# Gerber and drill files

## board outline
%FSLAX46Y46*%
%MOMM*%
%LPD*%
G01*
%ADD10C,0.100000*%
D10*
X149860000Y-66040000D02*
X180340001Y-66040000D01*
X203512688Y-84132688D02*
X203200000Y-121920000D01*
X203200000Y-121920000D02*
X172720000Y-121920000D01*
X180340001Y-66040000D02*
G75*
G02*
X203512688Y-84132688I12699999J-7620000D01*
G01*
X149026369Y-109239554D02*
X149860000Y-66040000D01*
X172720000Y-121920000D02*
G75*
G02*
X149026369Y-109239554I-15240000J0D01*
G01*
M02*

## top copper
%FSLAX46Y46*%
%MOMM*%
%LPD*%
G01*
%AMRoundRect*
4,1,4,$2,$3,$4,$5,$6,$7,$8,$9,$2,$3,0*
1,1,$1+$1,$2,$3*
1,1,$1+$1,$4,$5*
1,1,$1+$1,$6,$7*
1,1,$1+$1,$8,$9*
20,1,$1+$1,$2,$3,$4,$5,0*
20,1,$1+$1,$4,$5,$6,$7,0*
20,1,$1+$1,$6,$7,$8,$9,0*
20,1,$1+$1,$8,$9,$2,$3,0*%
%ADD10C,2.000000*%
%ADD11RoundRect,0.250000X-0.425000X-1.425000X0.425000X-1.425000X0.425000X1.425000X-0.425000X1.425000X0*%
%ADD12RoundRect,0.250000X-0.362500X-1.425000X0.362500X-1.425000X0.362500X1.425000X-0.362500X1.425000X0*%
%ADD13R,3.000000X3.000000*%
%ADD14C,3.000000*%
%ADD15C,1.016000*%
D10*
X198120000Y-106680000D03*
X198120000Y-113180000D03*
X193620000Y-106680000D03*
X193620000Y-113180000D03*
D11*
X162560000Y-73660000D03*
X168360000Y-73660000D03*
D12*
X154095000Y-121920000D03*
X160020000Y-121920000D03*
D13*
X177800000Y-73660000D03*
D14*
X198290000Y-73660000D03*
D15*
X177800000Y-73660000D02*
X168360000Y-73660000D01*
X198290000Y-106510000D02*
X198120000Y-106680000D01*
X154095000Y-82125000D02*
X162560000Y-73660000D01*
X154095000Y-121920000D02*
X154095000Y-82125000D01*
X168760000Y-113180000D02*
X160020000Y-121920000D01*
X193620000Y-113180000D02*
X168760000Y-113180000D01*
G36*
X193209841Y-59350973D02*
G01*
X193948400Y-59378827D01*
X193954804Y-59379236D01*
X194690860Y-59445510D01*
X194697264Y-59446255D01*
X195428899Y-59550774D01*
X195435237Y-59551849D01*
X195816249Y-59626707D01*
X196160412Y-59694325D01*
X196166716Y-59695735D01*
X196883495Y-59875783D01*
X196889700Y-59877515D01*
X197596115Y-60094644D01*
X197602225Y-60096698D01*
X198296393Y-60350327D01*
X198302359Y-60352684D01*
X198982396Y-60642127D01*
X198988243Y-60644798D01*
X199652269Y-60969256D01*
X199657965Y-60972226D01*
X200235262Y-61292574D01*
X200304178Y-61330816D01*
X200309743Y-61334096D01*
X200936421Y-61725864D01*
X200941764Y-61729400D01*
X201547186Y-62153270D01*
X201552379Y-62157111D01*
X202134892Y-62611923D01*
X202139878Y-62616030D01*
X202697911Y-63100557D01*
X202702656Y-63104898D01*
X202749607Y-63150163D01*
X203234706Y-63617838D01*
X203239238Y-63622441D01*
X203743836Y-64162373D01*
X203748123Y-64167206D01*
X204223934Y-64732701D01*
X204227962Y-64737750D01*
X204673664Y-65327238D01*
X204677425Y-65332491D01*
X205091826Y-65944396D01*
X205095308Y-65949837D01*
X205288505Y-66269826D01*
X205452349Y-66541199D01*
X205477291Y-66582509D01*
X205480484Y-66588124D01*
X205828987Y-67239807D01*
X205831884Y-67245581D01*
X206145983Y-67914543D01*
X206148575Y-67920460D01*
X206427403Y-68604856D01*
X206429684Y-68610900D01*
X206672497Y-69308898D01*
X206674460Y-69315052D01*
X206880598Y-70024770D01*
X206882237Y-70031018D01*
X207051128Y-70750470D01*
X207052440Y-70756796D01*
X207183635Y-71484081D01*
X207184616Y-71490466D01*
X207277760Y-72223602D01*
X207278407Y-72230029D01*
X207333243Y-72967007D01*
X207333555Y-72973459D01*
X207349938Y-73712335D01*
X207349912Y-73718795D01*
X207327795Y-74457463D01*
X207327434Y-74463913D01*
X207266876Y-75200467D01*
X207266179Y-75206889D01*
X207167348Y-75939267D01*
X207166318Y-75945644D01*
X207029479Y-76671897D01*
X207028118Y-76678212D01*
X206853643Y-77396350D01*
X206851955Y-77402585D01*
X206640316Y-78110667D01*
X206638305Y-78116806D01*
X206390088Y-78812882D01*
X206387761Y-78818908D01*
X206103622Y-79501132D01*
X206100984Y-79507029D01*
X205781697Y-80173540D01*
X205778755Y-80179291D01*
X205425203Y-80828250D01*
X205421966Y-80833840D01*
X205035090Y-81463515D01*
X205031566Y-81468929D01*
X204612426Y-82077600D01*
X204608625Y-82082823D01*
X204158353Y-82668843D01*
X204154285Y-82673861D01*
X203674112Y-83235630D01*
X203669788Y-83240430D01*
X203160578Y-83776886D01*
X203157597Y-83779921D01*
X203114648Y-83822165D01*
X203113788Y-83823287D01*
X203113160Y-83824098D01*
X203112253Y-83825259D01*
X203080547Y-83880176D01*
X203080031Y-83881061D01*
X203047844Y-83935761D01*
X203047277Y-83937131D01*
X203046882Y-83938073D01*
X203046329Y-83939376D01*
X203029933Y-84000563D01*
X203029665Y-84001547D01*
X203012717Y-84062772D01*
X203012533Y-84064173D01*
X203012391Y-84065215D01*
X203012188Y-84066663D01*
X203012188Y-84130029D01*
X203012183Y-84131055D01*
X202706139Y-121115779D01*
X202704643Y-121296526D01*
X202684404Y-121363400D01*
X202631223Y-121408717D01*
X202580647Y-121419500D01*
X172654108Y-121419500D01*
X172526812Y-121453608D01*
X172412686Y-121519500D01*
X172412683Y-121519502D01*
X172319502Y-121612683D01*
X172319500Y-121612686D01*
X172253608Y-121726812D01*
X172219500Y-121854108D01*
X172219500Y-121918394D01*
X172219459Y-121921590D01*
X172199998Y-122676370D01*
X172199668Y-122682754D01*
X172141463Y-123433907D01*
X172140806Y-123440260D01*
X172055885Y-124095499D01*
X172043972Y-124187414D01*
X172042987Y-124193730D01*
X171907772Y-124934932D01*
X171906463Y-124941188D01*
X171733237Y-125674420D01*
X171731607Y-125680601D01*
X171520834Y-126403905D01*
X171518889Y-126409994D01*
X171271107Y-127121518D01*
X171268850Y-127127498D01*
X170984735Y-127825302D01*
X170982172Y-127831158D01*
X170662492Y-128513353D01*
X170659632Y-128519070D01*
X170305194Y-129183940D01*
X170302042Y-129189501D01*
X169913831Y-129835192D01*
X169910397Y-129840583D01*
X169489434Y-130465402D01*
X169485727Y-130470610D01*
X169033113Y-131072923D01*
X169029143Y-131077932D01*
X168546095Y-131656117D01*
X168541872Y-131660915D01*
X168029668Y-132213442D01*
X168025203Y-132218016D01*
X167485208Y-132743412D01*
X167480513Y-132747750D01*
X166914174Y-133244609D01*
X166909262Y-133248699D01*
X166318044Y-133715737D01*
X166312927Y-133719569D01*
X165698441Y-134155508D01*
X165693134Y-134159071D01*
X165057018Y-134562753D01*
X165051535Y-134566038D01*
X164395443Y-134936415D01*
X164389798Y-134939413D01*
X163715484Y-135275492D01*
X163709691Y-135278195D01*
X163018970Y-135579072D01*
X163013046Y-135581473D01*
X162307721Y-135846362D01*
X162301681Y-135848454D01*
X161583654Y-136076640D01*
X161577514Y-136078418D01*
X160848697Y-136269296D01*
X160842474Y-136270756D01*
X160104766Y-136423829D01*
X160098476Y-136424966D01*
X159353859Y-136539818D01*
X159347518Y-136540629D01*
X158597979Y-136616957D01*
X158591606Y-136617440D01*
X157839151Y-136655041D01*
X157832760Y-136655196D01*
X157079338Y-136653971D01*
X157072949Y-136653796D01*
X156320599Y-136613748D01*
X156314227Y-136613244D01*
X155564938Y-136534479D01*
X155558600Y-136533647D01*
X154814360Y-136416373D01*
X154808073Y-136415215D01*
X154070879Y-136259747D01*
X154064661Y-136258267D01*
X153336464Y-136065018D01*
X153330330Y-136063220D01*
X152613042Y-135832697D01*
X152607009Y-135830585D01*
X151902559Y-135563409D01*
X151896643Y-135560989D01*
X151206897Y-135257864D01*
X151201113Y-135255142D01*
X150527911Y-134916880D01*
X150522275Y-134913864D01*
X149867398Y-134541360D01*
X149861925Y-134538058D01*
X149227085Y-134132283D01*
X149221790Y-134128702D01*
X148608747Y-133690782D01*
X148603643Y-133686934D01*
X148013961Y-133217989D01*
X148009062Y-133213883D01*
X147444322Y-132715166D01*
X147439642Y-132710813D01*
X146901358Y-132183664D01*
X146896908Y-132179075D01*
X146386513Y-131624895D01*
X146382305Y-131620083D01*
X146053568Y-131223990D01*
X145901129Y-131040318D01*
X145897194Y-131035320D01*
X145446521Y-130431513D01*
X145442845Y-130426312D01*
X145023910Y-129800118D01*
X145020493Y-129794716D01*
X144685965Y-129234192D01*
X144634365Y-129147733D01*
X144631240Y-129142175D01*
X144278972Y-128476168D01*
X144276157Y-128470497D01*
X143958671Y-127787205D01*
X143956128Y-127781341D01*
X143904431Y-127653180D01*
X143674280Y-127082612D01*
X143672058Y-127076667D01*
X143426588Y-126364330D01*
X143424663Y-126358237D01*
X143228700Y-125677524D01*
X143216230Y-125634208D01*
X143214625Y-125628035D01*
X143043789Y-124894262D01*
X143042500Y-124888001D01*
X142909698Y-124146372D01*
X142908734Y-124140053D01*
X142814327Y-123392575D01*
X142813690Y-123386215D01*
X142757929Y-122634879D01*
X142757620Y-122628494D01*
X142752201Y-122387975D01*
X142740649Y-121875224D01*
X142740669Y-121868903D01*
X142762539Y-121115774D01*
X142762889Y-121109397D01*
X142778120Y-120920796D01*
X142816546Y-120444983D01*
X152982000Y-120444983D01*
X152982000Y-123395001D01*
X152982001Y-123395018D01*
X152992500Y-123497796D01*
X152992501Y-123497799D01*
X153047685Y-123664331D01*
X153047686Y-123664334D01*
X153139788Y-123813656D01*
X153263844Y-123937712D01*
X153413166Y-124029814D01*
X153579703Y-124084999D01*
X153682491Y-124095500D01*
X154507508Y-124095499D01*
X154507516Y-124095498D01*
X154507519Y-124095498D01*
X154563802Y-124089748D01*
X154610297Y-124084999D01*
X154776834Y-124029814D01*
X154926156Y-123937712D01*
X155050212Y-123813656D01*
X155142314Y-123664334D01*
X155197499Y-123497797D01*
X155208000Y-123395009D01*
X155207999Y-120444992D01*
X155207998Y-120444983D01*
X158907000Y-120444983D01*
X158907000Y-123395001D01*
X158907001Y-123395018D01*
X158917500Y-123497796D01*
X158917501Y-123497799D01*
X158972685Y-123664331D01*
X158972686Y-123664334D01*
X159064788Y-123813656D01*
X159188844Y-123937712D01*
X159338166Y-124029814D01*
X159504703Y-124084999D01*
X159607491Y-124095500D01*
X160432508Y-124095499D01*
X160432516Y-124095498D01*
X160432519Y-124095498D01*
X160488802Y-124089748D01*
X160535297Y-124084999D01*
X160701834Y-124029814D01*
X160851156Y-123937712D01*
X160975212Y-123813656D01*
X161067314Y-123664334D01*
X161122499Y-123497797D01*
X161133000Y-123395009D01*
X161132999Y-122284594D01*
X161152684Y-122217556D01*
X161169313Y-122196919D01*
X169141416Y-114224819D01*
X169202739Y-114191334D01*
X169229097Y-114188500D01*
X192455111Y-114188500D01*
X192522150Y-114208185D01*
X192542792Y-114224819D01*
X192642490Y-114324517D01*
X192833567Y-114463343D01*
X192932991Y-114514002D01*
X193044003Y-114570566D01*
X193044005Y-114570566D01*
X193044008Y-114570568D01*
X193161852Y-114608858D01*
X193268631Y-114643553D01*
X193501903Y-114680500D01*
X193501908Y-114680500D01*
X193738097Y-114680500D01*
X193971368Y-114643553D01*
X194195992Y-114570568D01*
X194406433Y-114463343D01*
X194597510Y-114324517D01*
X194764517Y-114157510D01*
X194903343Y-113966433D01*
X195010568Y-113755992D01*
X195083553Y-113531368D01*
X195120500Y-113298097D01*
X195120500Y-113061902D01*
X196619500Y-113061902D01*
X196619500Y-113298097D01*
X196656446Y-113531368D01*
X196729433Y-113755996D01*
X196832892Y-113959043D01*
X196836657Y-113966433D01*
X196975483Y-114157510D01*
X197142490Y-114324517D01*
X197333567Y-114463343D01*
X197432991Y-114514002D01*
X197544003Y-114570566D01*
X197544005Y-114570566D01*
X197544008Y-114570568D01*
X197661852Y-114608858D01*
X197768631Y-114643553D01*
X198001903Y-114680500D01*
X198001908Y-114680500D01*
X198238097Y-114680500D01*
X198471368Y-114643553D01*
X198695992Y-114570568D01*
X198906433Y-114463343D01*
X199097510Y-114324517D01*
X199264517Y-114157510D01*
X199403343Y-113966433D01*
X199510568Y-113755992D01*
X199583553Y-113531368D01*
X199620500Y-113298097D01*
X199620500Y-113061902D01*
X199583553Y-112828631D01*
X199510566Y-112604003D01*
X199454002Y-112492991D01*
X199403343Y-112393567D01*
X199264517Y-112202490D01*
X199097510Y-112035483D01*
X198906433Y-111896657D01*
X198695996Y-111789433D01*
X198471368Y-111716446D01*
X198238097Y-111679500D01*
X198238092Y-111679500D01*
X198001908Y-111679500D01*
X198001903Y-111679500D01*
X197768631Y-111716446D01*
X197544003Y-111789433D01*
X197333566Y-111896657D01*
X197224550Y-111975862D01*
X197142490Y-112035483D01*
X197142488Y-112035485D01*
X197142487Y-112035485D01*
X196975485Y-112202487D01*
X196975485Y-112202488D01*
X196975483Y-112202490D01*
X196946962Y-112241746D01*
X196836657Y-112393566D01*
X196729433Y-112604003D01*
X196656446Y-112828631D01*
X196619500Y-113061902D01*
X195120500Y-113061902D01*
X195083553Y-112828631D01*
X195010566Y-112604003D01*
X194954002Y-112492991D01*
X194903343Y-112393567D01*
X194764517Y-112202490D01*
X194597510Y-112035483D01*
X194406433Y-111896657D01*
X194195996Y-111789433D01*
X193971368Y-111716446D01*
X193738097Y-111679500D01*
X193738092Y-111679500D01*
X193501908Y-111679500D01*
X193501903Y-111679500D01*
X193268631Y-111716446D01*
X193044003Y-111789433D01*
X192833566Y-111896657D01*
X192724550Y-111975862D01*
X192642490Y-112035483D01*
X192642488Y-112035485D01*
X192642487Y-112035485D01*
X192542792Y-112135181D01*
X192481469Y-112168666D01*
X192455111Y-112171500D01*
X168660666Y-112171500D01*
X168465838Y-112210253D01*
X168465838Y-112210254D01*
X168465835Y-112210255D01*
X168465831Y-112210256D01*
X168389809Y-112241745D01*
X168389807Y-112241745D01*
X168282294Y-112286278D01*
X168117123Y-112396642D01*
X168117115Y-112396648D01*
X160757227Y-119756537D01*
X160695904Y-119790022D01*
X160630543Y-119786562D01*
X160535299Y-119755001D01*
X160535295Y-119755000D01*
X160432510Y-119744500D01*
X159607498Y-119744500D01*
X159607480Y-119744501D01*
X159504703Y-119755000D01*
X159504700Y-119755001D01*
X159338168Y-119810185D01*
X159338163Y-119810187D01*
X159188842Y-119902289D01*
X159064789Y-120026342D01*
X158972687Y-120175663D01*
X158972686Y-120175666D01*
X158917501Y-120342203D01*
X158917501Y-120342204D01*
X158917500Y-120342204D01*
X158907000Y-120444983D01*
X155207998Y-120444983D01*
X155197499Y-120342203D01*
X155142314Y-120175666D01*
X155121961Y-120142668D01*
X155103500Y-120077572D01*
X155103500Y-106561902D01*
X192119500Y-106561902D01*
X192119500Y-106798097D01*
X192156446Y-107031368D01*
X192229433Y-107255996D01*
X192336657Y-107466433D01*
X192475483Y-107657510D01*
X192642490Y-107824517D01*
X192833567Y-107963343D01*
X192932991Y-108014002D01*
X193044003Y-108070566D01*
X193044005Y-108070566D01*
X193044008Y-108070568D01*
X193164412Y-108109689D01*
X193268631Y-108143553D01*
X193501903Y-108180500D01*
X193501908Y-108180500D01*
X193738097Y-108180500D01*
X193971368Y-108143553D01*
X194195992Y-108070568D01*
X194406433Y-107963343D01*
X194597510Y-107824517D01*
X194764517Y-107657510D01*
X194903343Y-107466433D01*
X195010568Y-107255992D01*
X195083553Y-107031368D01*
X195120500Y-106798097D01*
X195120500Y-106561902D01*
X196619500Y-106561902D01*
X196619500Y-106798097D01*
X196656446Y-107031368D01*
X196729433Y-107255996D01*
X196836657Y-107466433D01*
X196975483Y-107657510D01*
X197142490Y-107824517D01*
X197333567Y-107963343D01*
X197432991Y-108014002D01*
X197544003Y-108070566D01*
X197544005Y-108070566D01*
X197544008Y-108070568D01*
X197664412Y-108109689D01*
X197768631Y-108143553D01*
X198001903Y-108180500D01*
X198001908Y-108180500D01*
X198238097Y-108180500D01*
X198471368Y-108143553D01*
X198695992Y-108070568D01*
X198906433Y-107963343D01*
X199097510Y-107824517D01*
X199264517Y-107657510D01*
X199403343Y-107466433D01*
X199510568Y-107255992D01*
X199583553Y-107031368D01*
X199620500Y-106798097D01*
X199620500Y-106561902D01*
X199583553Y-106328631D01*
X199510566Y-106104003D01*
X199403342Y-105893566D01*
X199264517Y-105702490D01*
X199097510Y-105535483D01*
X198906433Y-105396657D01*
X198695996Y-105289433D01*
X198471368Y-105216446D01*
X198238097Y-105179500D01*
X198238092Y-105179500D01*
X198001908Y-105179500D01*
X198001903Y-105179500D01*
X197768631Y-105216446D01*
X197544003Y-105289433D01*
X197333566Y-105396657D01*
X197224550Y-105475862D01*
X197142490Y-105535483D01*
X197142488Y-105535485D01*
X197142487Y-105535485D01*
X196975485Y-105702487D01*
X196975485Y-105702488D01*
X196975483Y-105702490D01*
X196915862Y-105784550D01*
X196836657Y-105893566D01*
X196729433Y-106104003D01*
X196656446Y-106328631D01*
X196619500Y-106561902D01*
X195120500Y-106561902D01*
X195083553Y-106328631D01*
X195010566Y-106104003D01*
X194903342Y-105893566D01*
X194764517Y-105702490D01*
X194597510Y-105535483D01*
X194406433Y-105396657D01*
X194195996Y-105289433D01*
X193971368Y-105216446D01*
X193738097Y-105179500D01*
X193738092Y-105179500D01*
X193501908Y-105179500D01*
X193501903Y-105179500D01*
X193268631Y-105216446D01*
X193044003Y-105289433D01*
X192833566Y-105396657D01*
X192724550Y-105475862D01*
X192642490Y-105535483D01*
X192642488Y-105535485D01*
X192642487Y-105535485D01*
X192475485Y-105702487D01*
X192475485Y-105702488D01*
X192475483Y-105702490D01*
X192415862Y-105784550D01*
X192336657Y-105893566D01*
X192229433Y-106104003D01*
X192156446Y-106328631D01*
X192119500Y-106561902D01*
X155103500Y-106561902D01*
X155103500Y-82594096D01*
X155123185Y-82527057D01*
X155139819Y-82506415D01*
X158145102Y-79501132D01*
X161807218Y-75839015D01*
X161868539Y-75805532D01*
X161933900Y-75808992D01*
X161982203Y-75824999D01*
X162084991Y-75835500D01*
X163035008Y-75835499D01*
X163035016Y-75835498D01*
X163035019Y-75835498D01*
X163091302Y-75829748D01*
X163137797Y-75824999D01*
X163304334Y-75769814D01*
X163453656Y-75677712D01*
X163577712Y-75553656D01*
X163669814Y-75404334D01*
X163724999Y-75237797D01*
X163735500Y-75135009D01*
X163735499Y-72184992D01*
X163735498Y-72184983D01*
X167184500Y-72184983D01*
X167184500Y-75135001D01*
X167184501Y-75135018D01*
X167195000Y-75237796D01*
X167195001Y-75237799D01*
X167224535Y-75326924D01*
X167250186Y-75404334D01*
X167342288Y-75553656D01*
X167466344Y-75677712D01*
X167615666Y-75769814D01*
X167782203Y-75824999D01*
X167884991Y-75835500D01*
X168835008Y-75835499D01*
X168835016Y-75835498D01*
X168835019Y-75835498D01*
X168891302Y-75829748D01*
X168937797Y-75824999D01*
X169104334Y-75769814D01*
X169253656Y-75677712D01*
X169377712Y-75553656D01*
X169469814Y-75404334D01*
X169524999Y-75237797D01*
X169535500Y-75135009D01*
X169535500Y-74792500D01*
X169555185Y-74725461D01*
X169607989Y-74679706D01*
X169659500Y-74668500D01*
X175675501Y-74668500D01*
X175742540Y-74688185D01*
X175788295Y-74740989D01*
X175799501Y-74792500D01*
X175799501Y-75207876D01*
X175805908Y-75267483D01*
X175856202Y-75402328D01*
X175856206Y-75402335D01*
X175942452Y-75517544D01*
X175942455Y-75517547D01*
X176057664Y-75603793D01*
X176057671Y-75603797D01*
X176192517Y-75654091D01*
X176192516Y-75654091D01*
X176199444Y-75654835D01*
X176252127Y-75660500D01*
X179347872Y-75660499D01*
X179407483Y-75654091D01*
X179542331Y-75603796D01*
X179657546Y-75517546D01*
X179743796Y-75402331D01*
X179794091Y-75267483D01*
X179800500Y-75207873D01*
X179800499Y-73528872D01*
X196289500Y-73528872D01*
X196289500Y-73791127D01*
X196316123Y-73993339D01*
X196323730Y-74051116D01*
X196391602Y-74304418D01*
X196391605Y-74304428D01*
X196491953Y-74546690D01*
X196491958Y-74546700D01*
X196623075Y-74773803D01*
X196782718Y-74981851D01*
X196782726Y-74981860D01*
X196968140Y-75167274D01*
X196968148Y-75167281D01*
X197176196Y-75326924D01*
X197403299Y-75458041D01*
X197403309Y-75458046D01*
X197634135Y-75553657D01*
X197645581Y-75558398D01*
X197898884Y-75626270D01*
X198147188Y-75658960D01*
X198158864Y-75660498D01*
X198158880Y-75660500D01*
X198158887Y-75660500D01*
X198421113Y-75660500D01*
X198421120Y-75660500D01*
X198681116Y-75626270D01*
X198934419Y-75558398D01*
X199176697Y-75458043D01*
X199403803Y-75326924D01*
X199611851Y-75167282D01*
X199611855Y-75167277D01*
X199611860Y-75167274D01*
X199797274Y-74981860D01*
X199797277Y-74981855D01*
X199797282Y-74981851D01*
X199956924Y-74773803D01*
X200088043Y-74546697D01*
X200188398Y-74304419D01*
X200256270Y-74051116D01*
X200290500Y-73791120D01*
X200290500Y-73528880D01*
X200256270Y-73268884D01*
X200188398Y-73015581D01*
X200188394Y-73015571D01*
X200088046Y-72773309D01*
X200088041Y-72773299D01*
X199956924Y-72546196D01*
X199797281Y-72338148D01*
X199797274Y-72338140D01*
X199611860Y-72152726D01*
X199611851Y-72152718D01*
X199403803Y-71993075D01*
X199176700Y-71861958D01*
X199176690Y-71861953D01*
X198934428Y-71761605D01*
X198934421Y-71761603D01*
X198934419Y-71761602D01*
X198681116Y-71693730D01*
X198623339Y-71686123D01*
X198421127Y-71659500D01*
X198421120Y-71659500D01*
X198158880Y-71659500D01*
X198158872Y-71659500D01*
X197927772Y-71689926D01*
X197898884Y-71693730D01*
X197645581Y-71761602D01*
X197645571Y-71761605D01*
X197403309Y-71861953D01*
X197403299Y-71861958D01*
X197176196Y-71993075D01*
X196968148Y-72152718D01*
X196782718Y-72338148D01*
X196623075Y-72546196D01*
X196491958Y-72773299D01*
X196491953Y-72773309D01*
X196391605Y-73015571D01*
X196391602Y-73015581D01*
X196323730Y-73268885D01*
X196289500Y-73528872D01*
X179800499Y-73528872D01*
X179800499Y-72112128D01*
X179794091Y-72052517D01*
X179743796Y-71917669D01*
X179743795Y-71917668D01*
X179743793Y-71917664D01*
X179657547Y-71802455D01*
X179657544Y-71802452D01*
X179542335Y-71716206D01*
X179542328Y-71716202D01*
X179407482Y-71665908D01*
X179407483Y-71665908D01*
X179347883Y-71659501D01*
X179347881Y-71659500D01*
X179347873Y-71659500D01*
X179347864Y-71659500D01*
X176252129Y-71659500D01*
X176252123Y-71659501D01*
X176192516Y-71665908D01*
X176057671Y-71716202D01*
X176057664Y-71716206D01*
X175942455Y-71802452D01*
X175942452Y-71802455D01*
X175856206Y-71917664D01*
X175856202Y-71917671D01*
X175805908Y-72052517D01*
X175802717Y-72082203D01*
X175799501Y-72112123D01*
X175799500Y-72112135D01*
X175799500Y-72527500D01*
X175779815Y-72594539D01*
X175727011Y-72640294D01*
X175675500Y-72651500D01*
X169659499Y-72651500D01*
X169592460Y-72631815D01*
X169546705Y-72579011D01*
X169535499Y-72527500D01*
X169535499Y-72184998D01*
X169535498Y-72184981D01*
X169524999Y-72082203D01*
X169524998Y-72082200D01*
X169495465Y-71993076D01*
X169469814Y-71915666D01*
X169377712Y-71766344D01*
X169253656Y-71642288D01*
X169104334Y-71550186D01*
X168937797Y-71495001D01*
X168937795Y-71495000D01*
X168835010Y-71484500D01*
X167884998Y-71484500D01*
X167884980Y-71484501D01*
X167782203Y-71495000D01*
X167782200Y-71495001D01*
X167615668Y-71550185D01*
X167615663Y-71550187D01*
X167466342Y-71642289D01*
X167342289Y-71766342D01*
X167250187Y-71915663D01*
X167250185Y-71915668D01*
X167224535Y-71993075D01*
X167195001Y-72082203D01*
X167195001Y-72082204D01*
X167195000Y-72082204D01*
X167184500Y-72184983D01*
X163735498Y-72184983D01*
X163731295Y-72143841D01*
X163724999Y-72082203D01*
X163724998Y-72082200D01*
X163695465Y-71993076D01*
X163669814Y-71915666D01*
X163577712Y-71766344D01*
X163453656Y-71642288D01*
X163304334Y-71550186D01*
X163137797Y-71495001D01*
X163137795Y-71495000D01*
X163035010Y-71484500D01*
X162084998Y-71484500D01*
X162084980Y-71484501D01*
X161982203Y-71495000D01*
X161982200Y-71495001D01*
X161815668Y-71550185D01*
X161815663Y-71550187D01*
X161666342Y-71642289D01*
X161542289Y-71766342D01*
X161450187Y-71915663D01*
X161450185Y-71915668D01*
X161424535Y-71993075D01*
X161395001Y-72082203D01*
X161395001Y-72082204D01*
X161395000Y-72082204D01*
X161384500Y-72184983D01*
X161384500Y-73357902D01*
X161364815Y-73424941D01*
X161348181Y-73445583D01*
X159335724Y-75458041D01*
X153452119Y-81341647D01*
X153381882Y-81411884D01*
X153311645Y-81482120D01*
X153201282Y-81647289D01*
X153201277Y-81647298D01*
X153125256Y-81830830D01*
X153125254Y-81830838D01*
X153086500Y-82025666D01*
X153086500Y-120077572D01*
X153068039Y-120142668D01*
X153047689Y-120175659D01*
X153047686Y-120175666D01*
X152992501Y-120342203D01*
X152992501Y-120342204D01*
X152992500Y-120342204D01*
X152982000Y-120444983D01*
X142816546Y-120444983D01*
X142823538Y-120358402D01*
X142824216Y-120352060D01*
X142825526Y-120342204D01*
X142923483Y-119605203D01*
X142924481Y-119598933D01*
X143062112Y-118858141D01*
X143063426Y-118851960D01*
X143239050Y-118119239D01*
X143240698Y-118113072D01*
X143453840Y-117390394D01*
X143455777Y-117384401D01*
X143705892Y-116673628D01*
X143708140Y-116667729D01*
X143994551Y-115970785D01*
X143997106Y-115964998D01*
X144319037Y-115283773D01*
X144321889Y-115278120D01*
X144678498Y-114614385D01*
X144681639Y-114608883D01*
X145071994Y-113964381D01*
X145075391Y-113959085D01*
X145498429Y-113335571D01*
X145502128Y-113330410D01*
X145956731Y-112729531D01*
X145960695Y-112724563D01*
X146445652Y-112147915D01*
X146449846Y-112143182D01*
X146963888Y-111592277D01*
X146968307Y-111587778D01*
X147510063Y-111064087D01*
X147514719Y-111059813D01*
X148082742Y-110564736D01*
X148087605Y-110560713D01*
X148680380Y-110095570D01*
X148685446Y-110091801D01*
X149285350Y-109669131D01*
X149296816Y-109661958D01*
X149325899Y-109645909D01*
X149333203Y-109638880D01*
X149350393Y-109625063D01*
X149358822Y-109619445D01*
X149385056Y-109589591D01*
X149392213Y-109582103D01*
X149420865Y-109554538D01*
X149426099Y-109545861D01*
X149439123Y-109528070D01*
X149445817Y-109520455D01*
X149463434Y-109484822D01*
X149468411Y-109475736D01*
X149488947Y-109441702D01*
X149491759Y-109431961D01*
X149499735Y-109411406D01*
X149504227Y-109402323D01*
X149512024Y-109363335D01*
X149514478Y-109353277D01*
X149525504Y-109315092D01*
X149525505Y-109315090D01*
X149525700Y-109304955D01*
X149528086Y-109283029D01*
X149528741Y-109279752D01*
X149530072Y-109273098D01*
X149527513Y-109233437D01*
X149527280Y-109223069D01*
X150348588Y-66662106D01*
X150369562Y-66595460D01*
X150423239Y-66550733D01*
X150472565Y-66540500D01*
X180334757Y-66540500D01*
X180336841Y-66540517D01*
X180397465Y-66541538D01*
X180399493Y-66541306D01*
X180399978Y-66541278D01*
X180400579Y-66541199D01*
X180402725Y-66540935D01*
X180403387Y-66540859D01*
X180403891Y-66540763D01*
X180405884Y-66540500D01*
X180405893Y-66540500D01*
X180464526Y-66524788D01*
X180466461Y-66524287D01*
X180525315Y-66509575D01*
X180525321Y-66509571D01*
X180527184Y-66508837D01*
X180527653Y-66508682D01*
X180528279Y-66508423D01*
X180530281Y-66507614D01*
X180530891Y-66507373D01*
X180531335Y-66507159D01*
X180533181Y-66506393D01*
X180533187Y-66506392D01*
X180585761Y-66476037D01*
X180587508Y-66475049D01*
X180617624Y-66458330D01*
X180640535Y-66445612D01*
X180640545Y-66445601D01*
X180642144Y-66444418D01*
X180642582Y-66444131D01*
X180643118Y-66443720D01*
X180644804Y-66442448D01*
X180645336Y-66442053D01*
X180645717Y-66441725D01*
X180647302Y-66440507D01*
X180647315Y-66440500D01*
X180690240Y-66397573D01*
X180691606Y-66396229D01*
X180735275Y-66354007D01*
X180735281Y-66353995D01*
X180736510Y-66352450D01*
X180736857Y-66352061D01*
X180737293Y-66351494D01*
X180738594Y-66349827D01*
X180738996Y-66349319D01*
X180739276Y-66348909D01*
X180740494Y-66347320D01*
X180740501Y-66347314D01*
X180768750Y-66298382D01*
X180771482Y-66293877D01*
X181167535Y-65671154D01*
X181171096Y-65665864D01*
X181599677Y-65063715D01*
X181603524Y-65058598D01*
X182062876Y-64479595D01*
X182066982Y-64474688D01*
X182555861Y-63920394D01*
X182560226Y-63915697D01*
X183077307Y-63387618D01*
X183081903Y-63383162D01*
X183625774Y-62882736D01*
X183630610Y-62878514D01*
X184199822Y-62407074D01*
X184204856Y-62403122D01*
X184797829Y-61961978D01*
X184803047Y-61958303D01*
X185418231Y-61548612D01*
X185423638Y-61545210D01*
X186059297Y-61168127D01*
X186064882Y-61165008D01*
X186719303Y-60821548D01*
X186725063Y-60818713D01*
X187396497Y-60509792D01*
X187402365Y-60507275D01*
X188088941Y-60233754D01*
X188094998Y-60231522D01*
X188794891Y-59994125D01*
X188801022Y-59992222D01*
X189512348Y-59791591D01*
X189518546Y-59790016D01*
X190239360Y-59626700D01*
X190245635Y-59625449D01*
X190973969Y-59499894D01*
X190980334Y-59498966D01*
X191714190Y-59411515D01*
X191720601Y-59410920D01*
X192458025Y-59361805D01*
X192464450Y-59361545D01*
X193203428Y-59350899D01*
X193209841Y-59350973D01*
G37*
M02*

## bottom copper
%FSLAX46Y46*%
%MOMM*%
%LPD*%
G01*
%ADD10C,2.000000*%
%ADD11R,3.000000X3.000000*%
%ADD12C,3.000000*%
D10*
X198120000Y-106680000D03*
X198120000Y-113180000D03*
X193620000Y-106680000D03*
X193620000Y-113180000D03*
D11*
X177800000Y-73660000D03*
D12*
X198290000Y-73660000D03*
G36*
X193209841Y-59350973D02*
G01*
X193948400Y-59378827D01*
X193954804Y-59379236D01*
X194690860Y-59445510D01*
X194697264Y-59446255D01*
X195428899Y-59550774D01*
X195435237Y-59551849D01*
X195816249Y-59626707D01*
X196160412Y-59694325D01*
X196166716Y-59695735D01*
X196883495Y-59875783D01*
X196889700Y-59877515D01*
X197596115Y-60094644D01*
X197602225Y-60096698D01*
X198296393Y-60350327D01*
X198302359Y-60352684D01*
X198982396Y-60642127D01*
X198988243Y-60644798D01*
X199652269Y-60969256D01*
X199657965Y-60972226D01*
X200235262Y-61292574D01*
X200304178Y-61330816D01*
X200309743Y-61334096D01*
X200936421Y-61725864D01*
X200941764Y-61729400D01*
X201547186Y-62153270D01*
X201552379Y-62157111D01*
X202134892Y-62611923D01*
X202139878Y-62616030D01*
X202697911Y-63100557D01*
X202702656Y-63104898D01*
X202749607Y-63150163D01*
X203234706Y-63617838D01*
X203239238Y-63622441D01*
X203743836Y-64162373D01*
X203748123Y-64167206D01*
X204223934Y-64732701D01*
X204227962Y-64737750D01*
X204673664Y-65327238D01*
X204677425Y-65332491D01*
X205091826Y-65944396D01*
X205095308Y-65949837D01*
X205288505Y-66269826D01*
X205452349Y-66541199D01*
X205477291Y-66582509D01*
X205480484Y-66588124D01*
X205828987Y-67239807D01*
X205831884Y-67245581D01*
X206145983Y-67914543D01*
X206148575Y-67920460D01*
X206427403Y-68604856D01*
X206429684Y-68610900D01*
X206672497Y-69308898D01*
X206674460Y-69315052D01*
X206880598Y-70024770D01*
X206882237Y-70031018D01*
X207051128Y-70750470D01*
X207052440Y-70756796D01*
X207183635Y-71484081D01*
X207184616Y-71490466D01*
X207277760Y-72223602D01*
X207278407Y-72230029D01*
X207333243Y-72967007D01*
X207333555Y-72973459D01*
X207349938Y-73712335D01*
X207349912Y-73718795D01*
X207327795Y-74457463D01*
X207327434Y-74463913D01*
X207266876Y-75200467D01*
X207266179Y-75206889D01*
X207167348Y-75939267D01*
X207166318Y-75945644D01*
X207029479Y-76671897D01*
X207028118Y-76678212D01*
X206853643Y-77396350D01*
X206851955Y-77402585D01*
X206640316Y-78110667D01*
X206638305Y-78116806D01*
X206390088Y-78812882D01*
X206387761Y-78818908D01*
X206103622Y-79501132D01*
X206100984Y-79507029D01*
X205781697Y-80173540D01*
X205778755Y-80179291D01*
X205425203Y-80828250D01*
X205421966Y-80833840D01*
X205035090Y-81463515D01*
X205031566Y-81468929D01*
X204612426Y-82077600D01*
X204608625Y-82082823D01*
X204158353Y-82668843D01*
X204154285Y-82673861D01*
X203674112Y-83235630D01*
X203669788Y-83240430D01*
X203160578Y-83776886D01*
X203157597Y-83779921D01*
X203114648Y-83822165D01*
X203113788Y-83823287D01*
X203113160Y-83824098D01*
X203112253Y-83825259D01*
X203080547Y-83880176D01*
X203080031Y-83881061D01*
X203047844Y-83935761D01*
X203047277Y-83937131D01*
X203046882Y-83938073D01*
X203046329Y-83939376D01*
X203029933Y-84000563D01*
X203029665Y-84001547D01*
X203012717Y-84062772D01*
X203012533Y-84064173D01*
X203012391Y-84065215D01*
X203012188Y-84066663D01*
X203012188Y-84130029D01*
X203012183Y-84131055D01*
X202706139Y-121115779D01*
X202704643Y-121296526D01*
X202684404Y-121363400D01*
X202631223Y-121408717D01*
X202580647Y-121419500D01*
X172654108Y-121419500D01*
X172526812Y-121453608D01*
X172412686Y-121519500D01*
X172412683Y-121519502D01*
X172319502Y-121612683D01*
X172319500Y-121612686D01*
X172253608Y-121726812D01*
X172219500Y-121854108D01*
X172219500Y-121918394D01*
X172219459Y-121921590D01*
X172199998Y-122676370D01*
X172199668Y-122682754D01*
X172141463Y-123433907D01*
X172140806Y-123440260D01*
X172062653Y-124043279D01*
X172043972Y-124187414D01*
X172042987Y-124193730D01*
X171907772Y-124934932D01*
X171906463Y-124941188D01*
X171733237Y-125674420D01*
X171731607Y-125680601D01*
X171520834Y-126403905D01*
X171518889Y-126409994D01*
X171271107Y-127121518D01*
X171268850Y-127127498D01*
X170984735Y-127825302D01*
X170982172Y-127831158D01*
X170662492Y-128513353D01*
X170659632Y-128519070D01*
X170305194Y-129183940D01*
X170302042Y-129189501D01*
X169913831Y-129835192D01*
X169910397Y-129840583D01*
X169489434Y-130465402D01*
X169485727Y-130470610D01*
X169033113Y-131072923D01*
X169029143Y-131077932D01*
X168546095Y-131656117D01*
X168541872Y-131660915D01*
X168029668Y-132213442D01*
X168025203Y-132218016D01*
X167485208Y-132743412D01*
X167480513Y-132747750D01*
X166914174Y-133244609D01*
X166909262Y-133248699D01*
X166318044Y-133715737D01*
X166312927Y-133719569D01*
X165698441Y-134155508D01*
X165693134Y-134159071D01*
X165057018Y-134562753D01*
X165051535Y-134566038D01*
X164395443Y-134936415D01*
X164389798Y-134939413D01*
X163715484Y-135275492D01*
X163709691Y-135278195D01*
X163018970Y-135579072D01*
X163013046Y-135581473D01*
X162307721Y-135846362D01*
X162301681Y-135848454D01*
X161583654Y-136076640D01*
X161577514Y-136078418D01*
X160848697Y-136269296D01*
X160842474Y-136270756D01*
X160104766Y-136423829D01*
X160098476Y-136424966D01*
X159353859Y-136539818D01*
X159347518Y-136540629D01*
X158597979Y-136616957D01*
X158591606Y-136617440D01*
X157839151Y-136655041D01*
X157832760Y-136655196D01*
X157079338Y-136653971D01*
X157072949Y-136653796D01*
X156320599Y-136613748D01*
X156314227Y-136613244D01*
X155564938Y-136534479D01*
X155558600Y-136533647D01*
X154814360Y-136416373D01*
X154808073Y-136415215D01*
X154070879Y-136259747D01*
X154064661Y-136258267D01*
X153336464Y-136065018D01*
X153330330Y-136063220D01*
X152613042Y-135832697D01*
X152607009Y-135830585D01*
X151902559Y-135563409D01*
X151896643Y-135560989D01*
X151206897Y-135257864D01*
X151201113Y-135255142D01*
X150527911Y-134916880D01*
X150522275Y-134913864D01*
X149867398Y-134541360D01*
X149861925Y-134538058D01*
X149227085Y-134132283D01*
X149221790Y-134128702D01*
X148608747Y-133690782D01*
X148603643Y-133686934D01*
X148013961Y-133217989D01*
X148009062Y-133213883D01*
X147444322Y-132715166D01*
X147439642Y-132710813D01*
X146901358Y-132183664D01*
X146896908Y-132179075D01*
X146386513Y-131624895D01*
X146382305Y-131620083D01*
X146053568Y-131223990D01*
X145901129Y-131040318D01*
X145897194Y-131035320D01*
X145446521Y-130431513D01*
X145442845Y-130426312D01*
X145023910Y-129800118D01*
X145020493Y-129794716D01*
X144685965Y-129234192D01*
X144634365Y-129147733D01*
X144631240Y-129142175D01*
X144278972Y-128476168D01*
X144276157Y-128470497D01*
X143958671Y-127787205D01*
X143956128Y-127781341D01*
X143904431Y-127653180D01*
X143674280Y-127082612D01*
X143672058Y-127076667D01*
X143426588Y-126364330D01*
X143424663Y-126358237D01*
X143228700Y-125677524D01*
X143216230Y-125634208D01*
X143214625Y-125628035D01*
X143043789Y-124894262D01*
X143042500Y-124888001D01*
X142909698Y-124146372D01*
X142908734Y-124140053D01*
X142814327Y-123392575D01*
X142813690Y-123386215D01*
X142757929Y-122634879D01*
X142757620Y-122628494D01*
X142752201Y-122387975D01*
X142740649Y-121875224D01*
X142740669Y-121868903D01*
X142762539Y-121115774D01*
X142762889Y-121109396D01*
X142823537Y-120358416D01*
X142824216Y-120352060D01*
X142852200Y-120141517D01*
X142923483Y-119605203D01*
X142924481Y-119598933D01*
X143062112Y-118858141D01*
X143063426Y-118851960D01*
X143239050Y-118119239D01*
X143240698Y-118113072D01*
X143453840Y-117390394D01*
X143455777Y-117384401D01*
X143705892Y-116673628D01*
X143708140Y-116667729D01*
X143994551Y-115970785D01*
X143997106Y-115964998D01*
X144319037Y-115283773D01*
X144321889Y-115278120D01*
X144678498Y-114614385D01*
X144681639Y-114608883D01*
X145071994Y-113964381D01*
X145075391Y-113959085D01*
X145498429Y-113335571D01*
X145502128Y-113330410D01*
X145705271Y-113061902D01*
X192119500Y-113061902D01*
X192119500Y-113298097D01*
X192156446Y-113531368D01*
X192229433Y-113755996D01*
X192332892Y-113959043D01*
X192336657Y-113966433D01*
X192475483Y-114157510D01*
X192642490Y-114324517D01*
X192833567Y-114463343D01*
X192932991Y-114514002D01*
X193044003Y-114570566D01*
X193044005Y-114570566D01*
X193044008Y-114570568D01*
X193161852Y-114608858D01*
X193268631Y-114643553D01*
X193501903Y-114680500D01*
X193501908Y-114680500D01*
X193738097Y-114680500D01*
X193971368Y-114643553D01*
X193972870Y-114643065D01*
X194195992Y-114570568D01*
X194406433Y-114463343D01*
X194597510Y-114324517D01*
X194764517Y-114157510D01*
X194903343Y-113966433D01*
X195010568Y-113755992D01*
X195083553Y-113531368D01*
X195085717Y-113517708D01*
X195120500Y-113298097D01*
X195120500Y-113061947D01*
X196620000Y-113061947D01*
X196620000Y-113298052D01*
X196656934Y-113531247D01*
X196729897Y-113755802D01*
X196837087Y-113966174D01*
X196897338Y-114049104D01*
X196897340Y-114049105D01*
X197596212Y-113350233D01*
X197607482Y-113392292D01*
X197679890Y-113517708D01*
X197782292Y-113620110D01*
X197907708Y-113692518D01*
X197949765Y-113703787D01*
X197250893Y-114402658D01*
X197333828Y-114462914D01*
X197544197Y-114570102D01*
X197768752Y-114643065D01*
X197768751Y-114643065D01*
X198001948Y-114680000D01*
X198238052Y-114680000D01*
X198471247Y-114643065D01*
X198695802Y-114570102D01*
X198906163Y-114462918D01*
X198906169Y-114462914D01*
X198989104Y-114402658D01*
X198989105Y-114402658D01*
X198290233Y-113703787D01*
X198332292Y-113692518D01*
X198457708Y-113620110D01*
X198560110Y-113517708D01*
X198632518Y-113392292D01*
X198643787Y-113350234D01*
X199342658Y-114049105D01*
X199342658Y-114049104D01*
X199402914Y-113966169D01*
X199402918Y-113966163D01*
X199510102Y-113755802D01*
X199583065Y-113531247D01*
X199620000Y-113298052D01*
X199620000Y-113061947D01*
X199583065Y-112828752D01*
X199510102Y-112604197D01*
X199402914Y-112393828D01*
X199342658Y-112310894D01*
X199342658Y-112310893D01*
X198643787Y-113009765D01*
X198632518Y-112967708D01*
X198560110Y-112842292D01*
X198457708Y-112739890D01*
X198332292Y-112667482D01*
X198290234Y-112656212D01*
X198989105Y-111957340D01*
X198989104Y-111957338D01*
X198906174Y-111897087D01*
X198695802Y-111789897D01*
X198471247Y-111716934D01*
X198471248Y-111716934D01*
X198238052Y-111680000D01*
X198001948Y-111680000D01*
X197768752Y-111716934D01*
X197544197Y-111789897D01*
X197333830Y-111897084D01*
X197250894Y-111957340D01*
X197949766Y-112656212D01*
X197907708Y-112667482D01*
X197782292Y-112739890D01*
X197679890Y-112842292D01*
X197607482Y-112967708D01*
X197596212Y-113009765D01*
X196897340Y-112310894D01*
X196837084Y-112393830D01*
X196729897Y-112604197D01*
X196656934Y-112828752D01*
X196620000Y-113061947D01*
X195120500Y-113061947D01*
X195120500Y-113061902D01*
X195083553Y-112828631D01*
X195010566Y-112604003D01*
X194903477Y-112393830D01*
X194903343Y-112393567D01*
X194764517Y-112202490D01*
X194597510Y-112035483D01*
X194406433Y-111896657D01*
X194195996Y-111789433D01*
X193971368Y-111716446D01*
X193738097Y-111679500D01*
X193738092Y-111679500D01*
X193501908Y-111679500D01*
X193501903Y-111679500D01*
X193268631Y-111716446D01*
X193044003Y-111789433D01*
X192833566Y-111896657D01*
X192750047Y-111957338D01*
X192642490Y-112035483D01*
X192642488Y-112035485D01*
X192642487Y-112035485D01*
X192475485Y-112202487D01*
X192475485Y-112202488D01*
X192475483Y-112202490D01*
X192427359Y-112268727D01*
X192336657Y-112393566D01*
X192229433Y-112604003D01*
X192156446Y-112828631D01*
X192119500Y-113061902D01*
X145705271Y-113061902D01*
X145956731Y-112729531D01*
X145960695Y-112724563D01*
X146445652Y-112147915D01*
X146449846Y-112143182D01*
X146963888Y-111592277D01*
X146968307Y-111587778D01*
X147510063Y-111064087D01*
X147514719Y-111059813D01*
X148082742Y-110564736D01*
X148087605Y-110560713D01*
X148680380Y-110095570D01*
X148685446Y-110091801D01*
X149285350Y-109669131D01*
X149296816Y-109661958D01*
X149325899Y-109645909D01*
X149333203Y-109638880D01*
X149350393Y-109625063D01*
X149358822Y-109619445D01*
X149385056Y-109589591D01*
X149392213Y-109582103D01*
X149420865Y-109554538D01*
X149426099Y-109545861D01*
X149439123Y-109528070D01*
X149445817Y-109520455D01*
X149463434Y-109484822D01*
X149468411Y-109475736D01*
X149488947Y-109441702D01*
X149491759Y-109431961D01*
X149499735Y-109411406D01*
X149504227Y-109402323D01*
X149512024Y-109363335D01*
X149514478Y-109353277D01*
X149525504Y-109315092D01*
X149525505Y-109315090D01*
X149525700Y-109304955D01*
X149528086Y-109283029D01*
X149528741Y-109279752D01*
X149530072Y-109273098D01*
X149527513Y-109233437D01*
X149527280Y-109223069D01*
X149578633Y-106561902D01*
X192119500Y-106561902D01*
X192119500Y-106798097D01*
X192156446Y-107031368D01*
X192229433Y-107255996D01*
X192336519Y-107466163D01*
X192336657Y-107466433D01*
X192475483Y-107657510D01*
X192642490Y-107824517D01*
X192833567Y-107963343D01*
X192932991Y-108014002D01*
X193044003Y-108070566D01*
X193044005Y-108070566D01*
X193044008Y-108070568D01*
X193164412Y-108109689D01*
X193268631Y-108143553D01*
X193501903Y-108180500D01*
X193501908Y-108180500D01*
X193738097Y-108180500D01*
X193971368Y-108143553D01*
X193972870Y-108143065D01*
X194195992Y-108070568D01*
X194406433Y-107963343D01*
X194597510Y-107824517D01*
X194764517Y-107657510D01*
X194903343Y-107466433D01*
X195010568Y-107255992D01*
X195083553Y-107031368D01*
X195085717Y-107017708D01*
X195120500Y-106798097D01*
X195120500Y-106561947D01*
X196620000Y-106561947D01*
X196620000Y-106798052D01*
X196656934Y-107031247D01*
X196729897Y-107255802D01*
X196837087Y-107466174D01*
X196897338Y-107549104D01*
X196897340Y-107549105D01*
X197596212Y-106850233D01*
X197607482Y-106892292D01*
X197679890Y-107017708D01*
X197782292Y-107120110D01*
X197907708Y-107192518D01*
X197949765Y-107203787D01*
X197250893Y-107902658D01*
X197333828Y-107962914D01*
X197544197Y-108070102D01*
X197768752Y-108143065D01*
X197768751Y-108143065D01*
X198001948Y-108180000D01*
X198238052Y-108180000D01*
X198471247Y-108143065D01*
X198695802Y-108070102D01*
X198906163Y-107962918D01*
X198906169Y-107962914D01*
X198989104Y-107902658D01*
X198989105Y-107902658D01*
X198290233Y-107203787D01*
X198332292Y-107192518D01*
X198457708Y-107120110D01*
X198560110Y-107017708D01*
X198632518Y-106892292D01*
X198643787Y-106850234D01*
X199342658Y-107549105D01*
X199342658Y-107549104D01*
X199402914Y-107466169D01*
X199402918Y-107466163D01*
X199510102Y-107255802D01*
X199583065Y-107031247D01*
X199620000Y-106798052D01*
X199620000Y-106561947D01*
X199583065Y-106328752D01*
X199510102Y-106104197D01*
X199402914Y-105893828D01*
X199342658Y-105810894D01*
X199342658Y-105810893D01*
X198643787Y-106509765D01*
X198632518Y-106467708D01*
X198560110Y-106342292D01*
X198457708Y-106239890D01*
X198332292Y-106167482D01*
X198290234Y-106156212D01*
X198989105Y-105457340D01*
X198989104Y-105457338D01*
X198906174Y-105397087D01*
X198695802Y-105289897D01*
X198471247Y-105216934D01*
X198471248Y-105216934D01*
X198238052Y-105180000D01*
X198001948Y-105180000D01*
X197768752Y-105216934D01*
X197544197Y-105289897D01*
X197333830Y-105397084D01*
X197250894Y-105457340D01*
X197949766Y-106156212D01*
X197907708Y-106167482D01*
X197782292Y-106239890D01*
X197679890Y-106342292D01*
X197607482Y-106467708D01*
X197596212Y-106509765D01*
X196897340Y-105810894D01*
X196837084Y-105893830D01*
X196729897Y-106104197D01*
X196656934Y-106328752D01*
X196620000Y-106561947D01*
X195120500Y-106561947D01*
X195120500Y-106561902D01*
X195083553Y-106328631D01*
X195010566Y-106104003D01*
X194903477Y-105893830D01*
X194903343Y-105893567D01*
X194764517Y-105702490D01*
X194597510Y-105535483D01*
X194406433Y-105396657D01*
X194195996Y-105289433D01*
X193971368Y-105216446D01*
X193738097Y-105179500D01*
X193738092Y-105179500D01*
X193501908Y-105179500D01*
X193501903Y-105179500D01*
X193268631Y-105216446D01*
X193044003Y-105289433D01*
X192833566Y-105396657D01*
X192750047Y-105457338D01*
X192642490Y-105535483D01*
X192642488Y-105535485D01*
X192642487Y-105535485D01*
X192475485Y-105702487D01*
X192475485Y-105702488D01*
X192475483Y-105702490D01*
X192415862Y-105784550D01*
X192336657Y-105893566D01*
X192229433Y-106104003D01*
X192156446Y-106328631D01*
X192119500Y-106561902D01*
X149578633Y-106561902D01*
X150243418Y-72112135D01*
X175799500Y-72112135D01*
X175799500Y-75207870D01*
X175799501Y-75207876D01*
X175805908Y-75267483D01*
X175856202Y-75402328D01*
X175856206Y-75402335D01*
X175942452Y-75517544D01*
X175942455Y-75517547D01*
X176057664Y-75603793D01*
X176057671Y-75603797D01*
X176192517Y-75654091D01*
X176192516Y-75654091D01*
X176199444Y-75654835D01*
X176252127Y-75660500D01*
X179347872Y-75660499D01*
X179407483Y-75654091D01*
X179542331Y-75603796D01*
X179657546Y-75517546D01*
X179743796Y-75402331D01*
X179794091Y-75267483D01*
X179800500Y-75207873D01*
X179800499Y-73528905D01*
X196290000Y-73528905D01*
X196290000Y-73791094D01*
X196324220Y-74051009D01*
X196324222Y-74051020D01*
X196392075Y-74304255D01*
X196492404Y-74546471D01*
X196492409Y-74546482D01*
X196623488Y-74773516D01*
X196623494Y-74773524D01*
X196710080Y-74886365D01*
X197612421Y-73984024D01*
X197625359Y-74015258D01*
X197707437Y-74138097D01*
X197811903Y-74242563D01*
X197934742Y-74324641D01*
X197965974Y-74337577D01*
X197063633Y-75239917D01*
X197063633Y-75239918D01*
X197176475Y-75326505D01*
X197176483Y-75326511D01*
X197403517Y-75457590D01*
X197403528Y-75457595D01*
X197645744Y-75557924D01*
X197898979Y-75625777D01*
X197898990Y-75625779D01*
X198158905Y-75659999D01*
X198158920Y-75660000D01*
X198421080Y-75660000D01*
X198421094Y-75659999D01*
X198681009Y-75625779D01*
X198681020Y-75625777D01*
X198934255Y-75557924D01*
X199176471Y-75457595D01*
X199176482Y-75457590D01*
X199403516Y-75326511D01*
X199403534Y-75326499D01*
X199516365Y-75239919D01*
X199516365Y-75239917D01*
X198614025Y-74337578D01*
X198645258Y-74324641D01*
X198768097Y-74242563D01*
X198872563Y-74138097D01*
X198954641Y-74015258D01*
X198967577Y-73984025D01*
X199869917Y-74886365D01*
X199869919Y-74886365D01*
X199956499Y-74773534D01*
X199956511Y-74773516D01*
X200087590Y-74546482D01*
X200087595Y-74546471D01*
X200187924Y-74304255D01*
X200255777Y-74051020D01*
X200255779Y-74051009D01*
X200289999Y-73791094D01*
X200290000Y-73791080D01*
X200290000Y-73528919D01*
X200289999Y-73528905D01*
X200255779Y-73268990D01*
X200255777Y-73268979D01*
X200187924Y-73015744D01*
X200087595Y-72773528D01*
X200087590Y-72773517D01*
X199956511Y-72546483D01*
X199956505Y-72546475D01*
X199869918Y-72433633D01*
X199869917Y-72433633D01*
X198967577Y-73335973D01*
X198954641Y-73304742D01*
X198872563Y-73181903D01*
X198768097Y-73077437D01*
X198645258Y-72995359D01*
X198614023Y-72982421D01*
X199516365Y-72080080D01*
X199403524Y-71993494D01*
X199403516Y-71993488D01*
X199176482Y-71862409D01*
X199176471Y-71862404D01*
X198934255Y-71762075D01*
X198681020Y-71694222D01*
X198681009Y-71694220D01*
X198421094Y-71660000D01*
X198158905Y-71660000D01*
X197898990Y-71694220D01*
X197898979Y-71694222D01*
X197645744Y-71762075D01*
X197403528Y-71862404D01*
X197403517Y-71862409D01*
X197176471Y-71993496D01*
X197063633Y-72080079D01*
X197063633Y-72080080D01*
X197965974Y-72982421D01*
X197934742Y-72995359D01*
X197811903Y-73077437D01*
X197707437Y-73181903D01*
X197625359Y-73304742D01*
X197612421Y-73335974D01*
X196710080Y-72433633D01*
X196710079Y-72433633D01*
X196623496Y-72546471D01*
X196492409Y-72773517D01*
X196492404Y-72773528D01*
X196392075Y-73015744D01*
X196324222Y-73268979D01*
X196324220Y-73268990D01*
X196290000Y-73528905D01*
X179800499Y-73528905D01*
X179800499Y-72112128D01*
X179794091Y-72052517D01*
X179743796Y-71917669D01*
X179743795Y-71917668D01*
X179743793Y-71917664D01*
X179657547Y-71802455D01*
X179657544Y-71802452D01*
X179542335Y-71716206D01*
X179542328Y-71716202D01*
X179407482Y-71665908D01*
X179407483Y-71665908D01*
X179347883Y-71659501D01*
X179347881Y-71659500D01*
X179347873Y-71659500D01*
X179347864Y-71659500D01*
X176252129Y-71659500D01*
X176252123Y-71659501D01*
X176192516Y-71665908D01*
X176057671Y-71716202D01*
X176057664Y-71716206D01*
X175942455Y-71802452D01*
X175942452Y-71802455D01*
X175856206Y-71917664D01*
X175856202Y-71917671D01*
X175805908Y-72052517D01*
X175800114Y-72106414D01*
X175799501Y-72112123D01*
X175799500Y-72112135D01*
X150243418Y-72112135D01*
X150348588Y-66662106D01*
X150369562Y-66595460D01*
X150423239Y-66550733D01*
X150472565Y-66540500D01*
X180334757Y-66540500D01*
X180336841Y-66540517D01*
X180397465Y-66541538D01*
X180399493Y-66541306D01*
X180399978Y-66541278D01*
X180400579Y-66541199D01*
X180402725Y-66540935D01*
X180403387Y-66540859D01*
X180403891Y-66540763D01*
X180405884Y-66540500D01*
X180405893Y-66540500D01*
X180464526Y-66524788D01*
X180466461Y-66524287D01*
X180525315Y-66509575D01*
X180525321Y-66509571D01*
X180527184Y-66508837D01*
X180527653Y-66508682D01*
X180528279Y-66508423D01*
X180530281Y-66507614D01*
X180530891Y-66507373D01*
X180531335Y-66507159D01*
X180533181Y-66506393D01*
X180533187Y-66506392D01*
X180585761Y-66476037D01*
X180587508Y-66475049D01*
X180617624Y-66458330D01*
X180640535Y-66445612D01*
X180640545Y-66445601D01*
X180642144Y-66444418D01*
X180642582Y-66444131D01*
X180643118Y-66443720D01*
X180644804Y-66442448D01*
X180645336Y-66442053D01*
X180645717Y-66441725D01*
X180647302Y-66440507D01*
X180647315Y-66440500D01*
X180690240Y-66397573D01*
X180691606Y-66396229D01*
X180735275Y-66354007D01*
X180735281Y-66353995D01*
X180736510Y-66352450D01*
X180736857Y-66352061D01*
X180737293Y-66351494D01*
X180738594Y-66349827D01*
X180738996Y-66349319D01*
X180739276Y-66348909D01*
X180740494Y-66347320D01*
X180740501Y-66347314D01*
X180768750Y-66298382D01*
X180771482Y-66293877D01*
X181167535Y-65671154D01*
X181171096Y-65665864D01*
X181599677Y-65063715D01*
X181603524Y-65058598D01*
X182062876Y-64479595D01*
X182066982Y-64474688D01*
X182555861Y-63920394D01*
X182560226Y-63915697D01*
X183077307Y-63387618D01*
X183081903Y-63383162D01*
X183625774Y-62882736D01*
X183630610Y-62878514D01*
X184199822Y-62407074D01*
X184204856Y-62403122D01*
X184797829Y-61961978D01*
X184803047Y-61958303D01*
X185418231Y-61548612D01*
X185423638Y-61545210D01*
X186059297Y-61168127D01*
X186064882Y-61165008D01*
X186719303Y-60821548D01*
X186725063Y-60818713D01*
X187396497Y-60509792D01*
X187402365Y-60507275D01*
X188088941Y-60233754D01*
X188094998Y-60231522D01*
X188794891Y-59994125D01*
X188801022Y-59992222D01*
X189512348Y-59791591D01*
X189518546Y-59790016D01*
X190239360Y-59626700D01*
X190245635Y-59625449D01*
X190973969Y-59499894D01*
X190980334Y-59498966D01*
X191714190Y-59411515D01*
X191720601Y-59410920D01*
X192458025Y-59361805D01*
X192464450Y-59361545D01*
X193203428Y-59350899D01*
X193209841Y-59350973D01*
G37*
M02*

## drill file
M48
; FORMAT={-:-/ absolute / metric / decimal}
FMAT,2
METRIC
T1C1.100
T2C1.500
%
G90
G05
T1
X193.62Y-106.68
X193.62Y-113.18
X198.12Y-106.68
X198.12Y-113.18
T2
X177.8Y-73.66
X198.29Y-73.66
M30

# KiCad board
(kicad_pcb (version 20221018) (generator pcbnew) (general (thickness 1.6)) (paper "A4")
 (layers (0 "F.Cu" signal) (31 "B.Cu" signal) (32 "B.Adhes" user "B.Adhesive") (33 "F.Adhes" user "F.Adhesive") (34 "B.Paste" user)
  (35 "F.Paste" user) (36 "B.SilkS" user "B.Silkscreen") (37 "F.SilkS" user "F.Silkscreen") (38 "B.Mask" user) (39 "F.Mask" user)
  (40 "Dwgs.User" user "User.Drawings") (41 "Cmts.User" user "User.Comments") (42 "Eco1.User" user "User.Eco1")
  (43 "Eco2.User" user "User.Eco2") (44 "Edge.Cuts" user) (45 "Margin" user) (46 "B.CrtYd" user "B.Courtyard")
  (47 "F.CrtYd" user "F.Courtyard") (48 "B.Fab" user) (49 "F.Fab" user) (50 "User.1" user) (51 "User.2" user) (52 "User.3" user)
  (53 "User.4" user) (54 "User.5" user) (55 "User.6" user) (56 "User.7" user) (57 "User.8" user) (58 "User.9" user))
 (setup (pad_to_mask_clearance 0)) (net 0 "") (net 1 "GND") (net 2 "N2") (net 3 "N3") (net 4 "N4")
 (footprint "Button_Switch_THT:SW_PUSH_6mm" (layer "F.Cu") (at 198.12 106.68 -90)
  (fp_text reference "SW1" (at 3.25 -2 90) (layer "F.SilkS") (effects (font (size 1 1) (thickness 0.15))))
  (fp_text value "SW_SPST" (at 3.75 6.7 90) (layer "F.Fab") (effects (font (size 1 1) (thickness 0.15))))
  (pad "1" thru_hole circle (at 0 0) (size 2 2) (drill 1.1) (layers "*.Cu" "*.Mask") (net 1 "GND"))
  (pad "1" thru_hole circle (at 6.5 0) (size 2 2) (drill 1.1) (layers "*.Cu" "*.Mask") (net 1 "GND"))
  (pad "2" thru_hole circle (at 0 4.5) (size 2 2) (drill 1.1) (layers "*.Cu" "*.Mask") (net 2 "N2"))
  (pad "2" thru_hole circle (at 6.5 4.5) (size 2 2) (drill 1.1) (layers "*.Cu" "*.Mask") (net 2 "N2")))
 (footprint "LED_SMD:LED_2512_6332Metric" (layer "F.Cu") (at 165.46 73.66)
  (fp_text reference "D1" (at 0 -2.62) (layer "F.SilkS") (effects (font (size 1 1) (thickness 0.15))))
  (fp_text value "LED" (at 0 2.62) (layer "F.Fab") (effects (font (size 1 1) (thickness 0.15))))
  (pad "1" smd roundrect (at -2.9 0) (size 1.35 3.35) (layers "F.Cu" "F.Paste" "F.Mask") (roundrect_rratio 0.185185) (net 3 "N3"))
  (pad "2" smd roundrect (at 2.9 0) (size 1.35 3.35) (layers "F.Cu" "F.Paste" "F.Mask") (roundrect_rratio 0.185185) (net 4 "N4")))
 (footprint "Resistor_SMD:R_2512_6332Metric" (layer "F.Cu") (at 157.0575 121.92)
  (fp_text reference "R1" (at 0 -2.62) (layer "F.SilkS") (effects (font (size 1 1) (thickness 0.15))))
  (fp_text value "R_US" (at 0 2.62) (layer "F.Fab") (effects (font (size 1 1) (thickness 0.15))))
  (pad "1" smd roundrect (at -2.9625 0) (size 1.225 3.35) (layers "F.Cu" "F.Paste" "F.Mask") (roundrect_rratio 0.204082) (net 3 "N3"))
  (pad "2" smd roundrect (at 2.9625 0) (size 1.225 3.35) (layers "F.Cu" "F.Paste" "F.Mask") (roundrect_rratio 0.204082) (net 2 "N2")))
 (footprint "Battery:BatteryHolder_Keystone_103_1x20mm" (layer "F.Cu") (at 177.8 73.66)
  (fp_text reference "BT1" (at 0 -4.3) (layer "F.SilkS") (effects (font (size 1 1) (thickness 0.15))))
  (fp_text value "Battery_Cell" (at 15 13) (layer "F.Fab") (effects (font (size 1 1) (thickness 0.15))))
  (pad "1" thru_hole rect (at 0 0) (size 3 3) (drill 1.5) (layers "*.Cu" "*.Mask") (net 4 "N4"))
  (pad "2" thru_hole circle (at 20.49 0) (size 3 3) (drill 1.5) (layers "*.Cu" "*.Mask") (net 1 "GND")))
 (gr_line (start 149.86 66.04) (end 180.340001 66.04) (stroke (width 0.1) (type default)) (layer "Edge.Cuts"))
 (gr_line (start 203.512688 84.132688) (end 203.2 121.92) (stroke (width 0.1) (type default)) (layer "Edge.Cuts"))
 (gr_line (start 203.2 121.92) (end 172.72 121.92) (stroke (width 0.1) (type default)) (layer "Edge.Cuts"))
 (gr_arc (start 180.340001 66.04) (mid 202.154635 61.986191) (end 203.512688 84.132688) (stroke (width 0.1) (type default))
  (layer "Edge.Cuts"))
 (gr_line (start 149.026369 109.239554) (end 149.86 66.04) (stroke (width 0.1) (type default)) (layer "Edge.Cuts"))
 (gr_arc (start 172.72 121.92) (mid 150.288885 135.356721) (end 149.026369 109.239554) (stroke (width 0.1) (type default))
  (layer "Edge.Cuts"))
 (segment (start 177.8 73.66) (end 168.36 73.66) (width 1.016) (layer "F.Cu") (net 4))
 (segment (start 198.29 106.51) (end 198.12 106.68) (width 1.016) (layer "F.Cu") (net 1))
 (segment (start 154.095 82.125) (end 162.56 73.66) (width 1.016) (layer "F.Cu") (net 3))
 (segment (start 154.095 121.92) (end 154.095 82.125) (width 1.016) (layer "F.Cu") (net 3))
 (segment (start 168.76 113.18) (end 160.02 121.92) (width 1.016) (layer "F.Cu") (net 2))
 (segment (start 193.62 113.18) (end 168.76 113.18) (width 1.016) (layer "F.Cu") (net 2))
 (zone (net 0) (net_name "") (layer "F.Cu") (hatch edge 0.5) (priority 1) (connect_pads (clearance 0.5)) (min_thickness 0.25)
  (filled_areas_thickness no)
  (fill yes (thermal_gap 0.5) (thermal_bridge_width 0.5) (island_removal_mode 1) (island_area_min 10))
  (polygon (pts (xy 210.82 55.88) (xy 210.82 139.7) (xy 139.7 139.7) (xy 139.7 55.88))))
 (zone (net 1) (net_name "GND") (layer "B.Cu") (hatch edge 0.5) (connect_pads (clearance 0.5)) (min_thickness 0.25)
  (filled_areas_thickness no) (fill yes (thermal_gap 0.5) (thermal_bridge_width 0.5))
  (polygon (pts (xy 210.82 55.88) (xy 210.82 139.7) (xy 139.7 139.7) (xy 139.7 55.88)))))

